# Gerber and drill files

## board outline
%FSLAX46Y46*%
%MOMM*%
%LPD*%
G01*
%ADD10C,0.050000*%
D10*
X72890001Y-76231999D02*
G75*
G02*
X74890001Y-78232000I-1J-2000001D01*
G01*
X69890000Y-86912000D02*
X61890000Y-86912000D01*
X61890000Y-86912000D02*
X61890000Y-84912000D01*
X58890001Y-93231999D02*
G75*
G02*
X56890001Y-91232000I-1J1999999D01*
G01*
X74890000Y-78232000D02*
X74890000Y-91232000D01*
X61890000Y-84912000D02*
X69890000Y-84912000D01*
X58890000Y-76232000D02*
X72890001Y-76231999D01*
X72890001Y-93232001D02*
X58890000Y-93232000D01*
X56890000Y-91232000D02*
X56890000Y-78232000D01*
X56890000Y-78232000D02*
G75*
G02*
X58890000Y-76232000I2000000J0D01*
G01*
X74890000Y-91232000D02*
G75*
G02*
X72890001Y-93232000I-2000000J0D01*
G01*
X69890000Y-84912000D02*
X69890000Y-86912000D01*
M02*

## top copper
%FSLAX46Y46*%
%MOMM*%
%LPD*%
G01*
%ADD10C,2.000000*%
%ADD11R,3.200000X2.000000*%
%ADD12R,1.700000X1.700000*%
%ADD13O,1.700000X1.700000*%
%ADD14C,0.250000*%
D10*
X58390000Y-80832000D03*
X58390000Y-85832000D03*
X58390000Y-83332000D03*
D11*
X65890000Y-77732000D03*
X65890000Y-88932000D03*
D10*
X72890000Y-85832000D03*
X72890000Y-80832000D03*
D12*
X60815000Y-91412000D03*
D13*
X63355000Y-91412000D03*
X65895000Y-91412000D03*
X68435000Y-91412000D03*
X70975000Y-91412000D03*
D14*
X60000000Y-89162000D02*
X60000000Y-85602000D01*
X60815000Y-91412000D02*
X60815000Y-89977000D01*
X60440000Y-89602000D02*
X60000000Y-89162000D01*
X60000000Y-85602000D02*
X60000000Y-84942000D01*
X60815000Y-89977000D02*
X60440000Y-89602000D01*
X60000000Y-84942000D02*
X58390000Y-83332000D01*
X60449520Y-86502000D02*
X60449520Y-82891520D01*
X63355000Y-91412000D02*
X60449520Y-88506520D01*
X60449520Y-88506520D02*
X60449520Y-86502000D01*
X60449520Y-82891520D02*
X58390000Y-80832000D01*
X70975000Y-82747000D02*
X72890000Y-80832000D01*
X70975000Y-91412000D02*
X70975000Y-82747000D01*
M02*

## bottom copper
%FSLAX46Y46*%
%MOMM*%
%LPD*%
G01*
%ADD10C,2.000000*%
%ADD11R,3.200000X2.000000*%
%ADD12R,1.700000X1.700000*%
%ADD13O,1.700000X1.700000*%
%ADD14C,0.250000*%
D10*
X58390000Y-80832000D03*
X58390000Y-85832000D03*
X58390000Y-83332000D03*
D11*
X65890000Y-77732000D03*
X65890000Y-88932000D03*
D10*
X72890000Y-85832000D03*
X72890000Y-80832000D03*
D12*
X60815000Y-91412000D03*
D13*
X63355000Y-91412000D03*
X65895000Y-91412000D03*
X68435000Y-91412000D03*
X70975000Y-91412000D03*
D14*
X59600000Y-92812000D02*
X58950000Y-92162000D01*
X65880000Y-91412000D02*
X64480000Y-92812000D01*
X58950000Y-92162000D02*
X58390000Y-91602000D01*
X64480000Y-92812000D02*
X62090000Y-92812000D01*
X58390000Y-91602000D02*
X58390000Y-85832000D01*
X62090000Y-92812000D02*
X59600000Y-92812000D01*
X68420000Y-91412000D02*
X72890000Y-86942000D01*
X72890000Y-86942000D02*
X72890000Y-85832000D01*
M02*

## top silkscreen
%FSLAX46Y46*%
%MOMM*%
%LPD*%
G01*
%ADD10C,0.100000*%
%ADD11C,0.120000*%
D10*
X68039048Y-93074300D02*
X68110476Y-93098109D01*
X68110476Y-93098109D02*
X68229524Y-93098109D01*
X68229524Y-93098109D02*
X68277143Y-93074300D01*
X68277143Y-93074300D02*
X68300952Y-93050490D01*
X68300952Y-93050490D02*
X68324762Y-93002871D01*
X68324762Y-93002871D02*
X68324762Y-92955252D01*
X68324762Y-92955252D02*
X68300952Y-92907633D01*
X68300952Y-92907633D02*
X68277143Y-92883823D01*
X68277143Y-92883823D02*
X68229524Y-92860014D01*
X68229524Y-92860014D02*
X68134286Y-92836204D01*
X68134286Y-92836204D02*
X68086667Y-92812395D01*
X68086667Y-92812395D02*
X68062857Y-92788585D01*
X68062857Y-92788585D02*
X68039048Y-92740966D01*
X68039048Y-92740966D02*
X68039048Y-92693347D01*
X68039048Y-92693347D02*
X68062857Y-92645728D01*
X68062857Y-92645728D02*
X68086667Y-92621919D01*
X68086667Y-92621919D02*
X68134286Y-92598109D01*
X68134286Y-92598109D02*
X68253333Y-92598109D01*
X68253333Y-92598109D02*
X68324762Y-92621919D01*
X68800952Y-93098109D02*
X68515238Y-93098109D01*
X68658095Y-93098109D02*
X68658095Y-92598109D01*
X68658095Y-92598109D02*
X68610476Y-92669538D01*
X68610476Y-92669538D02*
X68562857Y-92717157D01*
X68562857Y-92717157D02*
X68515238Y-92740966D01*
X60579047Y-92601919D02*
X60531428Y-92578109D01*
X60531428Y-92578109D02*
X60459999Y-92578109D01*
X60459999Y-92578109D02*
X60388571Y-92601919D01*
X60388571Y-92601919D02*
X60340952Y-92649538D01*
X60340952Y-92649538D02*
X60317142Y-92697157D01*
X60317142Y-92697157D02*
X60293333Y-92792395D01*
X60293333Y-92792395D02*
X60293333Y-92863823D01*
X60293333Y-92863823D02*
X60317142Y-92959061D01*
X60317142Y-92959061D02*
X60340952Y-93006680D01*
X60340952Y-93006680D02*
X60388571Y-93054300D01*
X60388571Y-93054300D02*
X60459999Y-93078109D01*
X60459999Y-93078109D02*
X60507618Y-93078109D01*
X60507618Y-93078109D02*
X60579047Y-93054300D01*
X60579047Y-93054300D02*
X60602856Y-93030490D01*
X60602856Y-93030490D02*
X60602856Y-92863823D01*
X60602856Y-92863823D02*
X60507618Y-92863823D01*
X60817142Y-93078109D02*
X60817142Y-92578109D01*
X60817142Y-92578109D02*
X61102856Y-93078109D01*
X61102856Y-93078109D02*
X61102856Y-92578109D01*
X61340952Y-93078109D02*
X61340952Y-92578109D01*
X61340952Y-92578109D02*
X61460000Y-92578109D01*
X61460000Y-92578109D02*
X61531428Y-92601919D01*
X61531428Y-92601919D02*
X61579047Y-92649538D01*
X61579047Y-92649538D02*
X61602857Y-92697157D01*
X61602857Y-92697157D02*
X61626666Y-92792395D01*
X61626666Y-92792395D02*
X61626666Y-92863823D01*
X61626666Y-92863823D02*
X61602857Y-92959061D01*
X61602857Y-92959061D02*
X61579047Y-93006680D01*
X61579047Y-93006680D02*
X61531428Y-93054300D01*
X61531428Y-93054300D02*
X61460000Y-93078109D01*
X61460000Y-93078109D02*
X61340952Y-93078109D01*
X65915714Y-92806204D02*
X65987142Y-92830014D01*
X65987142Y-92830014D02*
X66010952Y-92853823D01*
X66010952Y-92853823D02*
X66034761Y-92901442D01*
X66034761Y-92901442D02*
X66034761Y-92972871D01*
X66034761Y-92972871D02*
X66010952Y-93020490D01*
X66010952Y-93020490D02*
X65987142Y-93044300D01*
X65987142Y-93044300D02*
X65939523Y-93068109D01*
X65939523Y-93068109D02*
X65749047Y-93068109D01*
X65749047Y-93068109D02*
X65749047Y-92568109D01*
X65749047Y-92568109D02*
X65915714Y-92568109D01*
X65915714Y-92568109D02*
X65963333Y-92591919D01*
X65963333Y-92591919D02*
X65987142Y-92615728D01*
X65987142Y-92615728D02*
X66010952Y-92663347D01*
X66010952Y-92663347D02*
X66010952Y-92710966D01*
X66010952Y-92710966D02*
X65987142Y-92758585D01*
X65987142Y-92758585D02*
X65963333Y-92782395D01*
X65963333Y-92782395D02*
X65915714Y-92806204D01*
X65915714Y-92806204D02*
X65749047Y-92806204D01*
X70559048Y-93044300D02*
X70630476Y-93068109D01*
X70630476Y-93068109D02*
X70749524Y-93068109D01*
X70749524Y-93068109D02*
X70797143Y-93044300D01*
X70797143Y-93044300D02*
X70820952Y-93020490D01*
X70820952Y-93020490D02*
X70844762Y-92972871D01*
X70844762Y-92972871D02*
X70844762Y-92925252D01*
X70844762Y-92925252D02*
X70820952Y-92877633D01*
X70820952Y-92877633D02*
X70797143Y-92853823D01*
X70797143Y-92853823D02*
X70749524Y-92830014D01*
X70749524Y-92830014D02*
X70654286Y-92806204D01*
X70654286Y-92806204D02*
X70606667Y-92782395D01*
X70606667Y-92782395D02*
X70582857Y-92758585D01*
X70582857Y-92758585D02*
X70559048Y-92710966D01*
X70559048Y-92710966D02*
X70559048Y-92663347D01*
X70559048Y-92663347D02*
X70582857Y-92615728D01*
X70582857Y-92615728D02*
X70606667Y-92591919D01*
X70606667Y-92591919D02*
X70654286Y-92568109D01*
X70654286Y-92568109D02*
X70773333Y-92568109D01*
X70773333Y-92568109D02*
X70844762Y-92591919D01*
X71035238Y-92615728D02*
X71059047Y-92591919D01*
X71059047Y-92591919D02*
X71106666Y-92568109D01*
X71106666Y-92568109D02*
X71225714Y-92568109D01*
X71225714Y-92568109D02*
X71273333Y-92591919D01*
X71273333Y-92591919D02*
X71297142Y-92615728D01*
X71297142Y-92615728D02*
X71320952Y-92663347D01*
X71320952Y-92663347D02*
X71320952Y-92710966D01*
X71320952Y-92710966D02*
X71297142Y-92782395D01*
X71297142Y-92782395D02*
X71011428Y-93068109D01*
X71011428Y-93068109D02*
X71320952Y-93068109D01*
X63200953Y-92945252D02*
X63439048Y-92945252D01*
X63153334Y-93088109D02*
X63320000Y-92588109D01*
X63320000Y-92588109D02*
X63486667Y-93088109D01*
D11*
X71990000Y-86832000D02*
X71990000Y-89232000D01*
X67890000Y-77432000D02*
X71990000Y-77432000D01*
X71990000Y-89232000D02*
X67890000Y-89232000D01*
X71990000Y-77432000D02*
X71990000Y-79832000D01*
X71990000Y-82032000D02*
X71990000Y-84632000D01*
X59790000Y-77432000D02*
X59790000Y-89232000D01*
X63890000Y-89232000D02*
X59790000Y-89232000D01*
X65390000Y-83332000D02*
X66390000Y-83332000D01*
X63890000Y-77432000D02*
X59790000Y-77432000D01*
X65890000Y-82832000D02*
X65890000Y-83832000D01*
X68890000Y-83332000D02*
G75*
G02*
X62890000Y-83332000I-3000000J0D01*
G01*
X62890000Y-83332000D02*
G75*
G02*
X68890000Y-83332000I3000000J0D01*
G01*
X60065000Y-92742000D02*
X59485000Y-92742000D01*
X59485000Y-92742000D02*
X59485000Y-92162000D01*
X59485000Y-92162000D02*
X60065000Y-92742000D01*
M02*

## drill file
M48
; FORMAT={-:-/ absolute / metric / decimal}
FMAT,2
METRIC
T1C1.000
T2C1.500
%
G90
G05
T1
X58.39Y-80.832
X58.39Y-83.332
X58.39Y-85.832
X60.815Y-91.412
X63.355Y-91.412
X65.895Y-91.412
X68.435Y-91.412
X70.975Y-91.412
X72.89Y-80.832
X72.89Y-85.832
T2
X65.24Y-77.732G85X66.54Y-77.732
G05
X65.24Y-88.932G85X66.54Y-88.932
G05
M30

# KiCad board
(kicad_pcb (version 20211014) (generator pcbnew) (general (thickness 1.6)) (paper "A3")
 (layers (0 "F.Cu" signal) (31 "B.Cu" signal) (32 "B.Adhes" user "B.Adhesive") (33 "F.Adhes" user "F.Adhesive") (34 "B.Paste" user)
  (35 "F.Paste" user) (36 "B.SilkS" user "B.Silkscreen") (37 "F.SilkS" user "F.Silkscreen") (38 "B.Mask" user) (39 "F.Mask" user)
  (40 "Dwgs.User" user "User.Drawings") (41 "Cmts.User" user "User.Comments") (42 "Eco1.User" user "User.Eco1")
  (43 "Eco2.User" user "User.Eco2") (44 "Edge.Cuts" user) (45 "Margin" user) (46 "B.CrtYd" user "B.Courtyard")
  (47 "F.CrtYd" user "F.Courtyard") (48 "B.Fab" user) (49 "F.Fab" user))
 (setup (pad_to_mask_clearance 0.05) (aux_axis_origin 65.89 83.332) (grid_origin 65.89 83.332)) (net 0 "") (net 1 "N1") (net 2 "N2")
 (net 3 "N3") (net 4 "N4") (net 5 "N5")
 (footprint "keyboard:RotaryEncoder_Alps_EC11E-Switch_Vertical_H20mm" (layer "F.Cu") (at 65.89 83.332)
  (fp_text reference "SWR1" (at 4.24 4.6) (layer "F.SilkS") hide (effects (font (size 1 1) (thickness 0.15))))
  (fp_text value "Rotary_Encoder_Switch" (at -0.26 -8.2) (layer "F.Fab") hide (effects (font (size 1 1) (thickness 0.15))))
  (fp_line (start 6.1 3.5) (end 6.1 5.9) (layer "F.SilkS") (width 0.12))
  (fp_line (start 2 -5.9) (end 6.1 -5.9) (layer "F.SilkS") (width 0.12))
  (fp_line (start 6.1 5.9) (end 2 5.9) (layer "F.SilkS") (width 0.12))
  (fp_line (start 6.1 -5.9) (end 6.1 -3.5) (layer "F.SilkS") (width 0.12))
  (fp_line (start 6.1 -1.3) (end 6.1 1.3) (layer "F.SilkS") (width 0.12))
  (fp_line (start -6.1 -5.9) (end -6.1 5.9) (layer "F.SilkS") (width 0.12))
  (fp_line (start -2 5.9) (end -6.1 5.9) (layer "F.SilkS") (width 0.12))
  (fp_line (start -0.5 0) (end 0.5 0) (layer "F.SilkS") (width 0.12))
  (fp_line (start -2 -5.9) (end -6.1 -5.9) (layer "F.SilkS") (width 0.12))
  (fp_line (start 0 -0.5) (end 0 0.5) (layer "F.SilkS") (width 0.12))
  (fp_circle (center 0 0) (end 3 0) (layer "F.SilkS") (width 0.12) (fill none))
  (pad "A" thru_hole circle (at -7.5 -2.5) (size 2 2) (drill 1) (layers *.Cu *.Mask) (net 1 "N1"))
  (pad "B" thru_hole circle (at -7.5 2.5) (size 2 2) (drill 1) (layers *.Cu *.Mask) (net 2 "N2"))
  (pad "C" thru_hole circle (at -7.5 0) (size 2 2) (drill 1) (layers *.Cu *.Mask) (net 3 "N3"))
  (pad "MP" thru_hole rect (at 0 -5.6) (size 3.2 2) (drill oval 2.8 1.5) (layers *.Cu *.Mask))
  (pad "MP" thru_hole rect (at 0 5.6) (size 3.2 2) (drill oval 2.8 1.5) (layers *.Cu *.Mask))
  (pad "S1" thru_hole circle (at 7 2.5) (size 2 2) (drill 1) (layers *.Cu *.Mask) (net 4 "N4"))
  (pad "S2" thru_hole circle (at 7 -2.5) (size 2 2) (drill 1) (layers *.Cu *.Mask) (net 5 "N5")))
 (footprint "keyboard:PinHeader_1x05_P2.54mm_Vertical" (layer "F.Cu") (at 60.815 91.412 90)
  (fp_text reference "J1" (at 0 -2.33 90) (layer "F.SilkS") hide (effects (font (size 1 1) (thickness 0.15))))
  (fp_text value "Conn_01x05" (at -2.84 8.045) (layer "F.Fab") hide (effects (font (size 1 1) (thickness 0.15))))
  (fp_line (start -1.33 -0.75) (end -1.33 -1.33) (layer "F.SilkS") (width 0.12))
  (fp_line (start -1.33 -1.33) (end -0.75 -1.33) (layer "F.SilkS") (width 0.12))
  (fp_line (start -0.75 -1.33) (end -1.33 -0.75) (layer "F.SilkS") (width 0.12))
  (pad "1" thru_hole rect (at 0 0 90) (size 1.7 1.7) (drill 1) (layers *.Cu *.Mask) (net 3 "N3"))
  (pad "2" thru_hole oval (at 0 2.54 90) (size 1.7 1.7) (drill 1) (layers *.Cu *.Mask) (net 1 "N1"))
  (pad "3" thru_hole oval (at 0 5.08 90) (size 1.7 1.7) (drill 1) (layers *.Cu *.Mask) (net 2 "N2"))
  (pad "4" thru_hole oval (at 0 7.62 90) (size 1.7 1.7) (drill 1) (layers *.Cu *.Mask) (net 4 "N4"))
  (pad "5" thru_hole oval (at 0 10.16 90) (size 1.7 1.7) (drill 1) (layers *.Cu *.Mask) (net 5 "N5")))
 (gr_arc (start 72.890001 76.231999) (mid 74.304215 76.817785) (end 74.89 78.232) (layer "Edge.Cuts") (width 0.05))
 (gr_line (start 69.89 86.912) (end 61.89 86.912) (layer "Edge.Cuts") (width 0.05))
 (gr_line (start 61.89 86.912) (end 61.89 84.912) (layer "Edge.Cuts") (width 0.05))
 (gr_arc (start 58.890001 93.231999) (mid 57.475787 92.646214) (end 56.89 91.232) (layer "Edge.Cuts") (width 0.05))
 (gr_line (start 74.89 78.232) (end 74.89 91.232) (layer "Edge.Cuts") (width 0.05))
 (gr_line (start 61.89 84.912) (end 69.89 84.912) (layer "Edge.Cuts") (width 0.05))
 (gr_line (start 58.89 76.232) (end 72.890001 76.231999) (layer "Edge.Cuts") (width 0.05))
 (gr_line (start 72.890001 93.232001) (end 58.89 93.232) (layer "Edge.Cuts") (width 0.05))
 (gr_line (start 56.89 91.232) (end 56.89 78.232) (layer "Edge.Cuts") (width 0.05))
 (gr_arc (start 56.89 78.232) (mid 57.475786 76.817786) (end 58.89 76.232) (layer "Edge.Cuts") (width 0.05))
 (gr_arc (start 74.89 91.232) (mid 74.304215 92.646214) (end 72.890001 93.232001) (layer "Edge.Cuts") (width 0.05))
 (gr_line (start 69.89 84.912) (end 69.89 86.912) (layer "Edge.Cuts") (width 0.05))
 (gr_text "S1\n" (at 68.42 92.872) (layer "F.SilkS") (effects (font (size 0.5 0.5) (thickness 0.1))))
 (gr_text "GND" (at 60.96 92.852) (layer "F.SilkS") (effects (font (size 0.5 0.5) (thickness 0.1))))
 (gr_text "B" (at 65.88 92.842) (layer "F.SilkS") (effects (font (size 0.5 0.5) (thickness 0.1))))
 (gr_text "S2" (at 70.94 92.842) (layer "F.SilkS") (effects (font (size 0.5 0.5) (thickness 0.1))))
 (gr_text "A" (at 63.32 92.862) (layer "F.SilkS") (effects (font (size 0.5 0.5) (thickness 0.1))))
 (segment (start 60 89.162) (end 60 85.602) (width 0.25) (layer "F.Cu") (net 3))
 (segment (start 60.815 91.412) (end 60.815 89.977) (width 0.25) (layer "F.Cu") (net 3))
 (segment (start 60.44 89.602) (end 60 89.162) (width 0.25) (layer "F.Cu") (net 3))
 (segment (start 60 85.602) (end 60 84.942) (width 0.25) (layer "F.Cu") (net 3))
 (segment (start 60.815 89.977) (end 60.44 89.602) (width 0.25) (layer "F.Cu") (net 3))
 (segment (start 60 84.942) (end 58.39 83.332) (width 0.25) (layer "F.Cu") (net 3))
 (segment (start 60.44952 86.502) (end 60.44952 82.89152) (width 0.25) (layer "F.Cu") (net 1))
 (segment (start 63.355 91.412) (end 60.44952 88.50652) (width 0.25) (layer "F.Cu") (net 1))
 (segment (start 60.44952 88.50652) (end 60.44952 86.502) (width 0.25) (layer "F.Cu") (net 1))
 (segment (start 60.44952 82.89152) (end 58.39 80.832) (width 0.25) (layer "F.Cu") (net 1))
 (segment (start 59.6 92.812) (end 58.95 92.162) (width 0.25) (layer "B.Cu") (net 2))
 (segment (start 65.88 91.412) (end 64.48 92.812) (width 0.25) (layer "B.Cu") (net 2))
 (segment (start 58.95 92.162) (end 58.39 91.602) (width 0.25) (layer "B.Cu") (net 2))
 (segment (start 64.48 92.812) (end 62.09 92.812) (width 0.25) (layer "B.Cu") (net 2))
 (segment (start 58.39 91.602) (end 58.39 85.832) (width 0.25) (layer "B.Cu") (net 2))
 (segment (start 62.09 92.812) (end 59.6 92.812) (width 0.25) (layer "B.Cu") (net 2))
 (segment (start 68.42 91.412) (end 72.89 86.942) (width 0.25) (layer "B.Cu") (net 4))
 (segment (start 72.89 86.942) (end 72.89 85.832) (width 0.25) (layer "B.Cu") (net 4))
 (segment (start 70.975 82.747) (end 72.89 80.832) (width 0.25) (layer "F.Cu") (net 5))
 (segment (start 70.975 91.412) (end 70.975 82.747) (width 0.25) (layer "F.Cu") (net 5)))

